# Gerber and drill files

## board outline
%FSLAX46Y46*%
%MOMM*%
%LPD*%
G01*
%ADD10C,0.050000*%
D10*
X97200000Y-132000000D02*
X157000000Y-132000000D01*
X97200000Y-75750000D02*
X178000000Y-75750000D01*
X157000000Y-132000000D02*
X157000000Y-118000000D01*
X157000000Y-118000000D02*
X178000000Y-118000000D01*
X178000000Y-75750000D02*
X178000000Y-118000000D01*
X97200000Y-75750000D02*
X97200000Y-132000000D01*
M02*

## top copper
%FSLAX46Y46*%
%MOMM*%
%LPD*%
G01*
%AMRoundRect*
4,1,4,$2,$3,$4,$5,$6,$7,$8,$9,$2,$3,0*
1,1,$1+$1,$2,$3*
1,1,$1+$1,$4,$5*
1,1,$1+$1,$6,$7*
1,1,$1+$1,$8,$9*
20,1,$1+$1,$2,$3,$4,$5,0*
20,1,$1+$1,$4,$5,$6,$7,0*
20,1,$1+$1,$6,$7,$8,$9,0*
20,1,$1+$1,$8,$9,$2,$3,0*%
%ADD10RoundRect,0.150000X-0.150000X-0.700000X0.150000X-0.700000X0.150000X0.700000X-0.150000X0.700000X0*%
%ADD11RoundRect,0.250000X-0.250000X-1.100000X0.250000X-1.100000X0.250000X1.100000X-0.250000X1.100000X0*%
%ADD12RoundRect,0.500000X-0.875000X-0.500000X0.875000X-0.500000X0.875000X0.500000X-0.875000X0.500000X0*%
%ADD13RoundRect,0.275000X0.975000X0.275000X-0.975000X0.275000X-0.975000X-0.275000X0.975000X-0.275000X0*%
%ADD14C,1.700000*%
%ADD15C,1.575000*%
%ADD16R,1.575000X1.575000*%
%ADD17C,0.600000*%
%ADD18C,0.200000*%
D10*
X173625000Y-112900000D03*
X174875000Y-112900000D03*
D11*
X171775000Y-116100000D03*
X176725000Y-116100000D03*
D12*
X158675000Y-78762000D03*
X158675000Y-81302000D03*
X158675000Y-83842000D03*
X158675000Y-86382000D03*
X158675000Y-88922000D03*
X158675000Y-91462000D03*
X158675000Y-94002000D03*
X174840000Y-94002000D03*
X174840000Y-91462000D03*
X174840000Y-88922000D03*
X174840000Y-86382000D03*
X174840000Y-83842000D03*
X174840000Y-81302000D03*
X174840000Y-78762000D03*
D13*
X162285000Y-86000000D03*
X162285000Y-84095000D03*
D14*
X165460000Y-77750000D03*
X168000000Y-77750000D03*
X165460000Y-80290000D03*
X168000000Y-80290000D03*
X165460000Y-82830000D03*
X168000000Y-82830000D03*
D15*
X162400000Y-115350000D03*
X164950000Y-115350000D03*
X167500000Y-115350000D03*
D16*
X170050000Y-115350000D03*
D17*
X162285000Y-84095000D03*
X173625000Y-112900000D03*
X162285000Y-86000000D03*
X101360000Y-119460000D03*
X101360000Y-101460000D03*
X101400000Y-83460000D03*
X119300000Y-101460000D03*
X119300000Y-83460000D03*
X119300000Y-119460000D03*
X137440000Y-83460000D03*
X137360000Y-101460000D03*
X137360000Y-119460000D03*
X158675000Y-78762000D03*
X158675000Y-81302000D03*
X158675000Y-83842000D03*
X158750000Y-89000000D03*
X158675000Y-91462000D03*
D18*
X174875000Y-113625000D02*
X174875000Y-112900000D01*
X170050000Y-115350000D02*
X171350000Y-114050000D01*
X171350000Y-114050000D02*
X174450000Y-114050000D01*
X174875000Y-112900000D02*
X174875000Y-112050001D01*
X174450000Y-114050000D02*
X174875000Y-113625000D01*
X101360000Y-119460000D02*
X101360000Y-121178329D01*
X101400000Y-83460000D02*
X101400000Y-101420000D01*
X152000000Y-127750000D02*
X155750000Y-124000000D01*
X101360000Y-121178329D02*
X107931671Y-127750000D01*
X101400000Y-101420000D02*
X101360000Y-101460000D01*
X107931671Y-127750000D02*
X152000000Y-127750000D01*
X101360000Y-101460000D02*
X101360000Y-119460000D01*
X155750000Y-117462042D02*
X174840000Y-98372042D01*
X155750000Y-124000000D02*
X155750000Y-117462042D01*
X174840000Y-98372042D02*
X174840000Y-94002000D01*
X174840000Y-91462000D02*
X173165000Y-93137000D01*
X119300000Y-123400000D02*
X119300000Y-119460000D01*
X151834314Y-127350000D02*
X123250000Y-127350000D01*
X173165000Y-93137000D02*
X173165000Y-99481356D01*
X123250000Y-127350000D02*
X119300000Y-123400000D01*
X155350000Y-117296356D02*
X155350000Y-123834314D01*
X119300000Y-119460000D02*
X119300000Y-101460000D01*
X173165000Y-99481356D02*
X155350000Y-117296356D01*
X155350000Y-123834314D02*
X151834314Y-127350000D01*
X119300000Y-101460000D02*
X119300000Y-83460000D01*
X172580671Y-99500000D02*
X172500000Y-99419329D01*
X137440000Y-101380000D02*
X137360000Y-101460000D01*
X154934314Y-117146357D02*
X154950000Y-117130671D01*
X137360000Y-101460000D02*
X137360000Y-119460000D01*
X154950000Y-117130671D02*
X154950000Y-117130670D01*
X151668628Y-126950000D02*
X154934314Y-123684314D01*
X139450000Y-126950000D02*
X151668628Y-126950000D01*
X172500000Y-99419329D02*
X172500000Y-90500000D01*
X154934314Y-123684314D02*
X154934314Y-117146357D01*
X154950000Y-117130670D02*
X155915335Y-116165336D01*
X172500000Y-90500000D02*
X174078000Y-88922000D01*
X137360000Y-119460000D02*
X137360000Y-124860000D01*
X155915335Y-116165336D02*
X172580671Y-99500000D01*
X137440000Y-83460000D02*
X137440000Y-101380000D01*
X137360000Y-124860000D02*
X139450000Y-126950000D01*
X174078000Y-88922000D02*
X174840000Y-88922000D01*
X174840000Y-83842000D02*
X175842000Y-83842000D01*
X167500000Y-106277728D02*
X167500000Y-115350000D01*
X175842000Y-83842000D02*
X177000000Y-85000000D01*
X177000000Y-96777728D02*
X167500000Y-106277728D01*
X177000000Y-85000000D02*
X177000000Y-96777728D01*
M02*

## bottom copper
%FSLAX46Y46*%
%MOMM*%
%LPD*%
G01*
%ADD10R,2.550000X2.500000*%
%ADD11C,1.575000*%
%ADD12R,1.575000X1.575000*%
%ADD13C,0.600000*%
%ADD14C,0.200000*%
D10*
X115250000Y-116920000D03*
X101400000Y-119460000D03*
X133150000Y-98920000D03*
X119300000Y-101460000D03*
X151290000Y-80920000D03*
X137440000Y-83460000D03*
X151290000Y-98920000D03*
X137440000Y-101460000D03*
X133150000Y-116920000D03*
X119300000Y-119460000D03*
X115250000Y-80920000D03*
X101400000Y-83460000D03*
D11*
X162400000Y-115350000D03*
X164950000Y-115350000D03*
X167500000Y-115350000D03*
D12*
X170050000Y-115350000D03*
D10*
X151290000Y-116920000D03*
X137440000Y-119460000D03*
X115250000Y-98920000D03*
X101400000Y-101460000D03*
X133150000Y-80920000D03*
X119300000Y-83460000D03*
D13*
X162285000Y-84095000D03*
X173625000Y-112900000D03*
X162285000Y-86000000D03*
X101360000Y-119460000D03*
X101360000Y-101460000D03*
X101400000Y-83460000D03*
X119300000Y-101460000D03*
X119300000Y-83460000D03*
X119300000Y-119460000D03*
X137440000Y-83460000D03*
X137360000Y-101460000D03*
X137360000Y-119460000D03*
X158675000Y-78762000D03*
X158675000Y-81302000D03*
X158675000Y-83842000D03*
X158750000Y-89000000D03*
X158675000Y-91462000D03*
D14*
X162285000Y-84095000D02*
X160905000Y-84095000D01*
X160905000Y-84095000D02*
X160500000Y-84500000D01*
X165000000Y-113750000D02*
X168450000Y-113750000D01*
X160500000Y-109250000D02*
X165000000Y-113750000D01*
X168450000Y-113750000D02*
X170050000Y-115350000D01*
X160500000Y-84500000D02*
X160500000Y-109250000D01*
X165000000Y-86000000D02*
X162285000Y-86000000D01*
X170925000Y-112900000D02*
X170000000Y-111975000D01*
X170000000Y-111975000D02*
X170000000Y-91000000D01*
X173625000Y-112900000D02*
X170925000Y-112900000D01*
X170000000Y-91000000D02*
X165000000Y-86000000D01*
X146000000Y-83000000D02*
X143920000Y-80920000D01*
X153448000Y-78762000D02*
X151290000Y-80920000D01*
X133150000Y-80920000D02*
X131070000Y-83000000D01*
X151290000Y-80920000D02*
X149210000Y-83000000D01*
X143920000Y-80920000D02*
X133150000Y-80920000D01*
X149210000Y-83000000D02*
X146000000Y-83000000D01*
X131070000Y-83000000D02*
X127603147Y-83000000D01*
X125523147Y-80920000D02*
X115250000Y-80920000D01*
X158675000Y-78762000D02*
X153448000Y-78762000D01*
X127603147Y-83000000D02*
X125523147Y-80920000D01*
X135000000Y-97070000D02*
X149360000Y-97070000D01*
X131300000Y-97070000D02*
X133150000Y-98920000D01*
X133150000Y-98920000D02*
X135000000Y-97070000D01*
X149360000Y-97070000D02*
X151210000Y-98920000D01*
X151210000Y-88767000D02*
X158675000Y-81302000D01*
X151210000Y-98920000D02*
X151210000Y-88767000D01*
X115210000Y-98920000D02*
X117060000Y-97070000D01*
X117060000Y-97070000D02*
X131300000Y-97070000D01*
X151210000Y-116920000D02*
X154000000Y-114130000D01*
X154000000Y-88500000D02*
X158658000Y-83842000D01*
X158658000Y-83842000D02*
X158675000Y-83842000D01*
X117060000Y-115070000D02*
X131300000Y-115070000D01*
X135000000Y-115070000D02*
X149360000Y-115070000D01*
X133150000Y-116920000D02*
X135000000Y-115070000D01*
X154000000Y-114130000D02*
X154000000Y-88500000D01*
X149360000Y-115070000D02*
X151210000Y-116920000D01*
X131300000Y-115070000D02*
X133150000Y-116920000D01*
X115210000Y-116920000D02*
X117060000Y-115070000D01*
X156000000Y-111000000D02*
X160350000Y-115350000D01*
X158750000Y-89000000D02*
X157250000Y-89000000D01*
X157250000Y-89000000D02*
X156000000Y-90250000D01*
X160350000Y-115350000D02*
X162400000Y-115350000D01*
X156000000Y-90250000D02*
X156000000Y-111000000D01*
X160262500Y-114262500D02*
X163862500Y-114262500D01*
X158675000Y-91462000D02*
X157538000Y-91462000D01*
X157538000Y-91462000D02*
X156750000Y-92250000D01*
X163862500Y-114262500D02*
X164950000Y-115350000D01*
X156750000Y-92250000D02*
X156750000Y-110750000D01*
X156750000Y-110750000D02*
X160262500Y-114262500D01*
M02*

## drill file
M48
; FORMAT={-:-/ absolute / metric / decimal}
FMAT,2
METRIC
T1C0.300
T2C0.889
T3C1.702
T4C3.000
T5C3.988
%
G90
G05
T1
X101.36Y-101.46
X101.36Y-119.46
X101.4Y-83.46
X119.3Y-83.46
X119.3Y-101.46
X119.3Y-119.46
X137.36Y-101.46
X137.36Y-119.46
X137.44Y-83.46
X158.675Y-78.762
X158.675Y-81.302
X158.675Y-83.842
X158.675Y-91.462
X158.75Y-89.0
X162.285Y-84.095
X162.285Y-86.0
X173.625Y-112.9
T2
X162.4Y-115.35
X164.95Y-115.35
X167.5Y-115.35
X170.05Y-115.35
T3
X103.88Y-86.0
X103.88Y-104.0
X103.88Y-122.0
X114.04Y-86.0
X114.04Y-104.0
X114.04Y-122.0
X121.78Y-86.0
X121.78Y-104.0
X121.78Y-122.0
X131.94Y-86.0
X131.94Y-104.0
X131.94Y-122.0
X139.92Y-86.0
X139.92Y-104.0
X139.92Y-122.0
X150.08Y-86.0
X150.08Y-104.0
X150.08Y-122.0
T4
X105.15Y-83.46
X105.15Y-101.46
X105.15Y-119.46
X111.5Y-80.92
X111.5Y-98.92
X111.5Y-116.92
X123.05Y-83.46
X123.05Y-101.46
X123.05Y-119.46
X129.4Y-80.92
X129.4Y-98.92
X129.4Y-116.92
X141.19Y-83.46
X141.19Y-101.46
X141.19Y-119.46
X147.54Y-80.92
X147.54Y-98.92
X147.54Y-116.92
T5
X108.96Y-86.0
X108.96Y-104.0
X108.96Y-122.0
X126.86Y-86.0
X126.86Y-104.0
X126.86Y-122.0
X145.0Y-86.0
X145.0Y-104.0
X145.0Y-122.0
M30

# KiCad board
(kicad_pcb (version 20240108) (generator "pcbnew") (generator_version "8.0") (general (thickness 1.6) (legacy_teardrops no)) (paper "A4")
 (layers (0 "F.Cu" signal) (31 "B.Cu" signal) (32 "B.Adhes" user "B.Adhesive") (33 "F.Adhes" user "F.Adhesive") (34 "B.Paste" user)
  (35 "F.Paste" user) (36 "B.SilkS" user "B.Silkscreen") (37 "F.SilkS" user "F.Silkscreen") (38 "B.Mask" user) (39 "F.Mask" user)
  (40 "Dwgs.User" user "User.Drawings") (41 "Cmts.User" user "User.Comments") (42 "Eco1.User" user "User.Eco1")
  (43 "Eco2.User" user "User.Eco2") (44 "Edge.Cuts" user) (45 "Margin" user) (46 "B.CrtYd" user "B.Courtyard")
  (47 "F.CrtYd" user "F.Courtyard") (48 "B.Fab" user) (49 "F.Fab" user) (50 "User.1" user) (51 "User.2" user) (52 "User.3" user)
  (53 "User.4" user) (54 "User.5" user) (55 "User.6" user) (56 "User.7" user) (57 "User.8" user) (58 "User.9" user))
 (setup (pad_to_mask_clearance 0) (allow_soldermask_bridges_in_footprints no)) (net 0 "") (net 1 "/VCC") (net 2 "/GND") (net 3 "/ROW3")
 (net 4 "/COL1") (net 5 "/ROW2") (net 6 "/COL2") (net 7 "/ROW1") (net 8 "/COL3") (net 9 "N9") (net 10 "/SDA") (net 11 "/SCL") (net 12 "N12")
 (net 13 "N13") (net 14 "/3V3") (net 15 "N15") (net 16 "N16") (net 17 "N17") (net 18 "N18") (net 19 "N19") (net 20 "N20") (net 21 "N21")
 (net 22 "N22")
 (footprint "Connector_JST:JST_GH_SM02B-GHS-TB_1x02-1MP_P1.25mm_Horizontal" (layer "F.Cu") (at 174.25 114.75)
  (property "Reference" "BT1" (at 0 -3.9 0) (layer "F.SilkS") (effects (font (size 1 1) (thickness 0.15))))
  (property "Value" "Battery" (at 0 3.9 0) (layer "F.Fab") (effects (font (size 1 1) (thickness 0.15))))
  (pad "1" smd roundrect (at -0.625 -1.85) (size 0.6 1.7) (layers "F.Cu" "F.Paste" "F.Mask") (roundrect_rratio 0.25) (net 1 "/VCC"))
  (pad "2" smd roundrect (at 0.625 -1.85) (size 0.6 1.7) (layers "F.Cu" "F.Paste" "F.Mask") (roundrect_rratio 0.25) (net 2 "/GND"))
  (pad "MP" smd roundrect (at -2.475 1.35) (size 1 2.7) (layers "F.Cu" "F.Paste" "F.Mask") (roundrect_rratio 0.25))
  (pad "MP" smd roundrect (at 2.475 1.35) (size 1 2.7) (layers "F.Cu" "F.Paste" "F.Mask") (roundrect_rratio 0.25)))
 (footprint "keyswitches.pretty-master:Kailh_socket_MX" (layer "F.Cu") (at 108.96 122)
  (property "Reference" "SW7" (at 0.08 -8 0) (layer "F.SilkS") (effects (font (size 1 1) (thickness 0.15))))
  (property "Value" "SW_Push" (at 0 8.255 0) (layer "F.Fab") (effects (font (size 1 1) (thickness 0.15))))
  (pad "" np_thru_hole circle (at -5.08 0) (size 1.7018 1.7018) (drill 1.7018) (layers "*.Cu" "*.Mask"))
  (pad "" np_thru_hole circle (at -3.81 -2.54) (size 3 3) (drill 3) (layers "*.Cu" "*.Mask"))
  (pad "" np_thru_hole circle (at 0 0) (size 3.9878 3.9878) (drill 3.9878) (layers "*.Cu" "*.Mask"))
  (pad "" np_thru_hole circle (at 2.54 -5.08) (size 3 3) (drill 3) (layers "*.Cu" "*.Mask"))
  (pad "" np_thru_hole circle (at 5.08 0) (size 1.7018 1.7018) (drill 1.7018) (layers "*.Cu" "*.Mask"))
  (pad "1" smd rect (at 6.29 -5.08) (size 2.55 2.5) (layers "B.Cu" "B.Paste" "B.Mask") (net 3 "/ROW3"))
  (pad "2" smd rect (at -7.56 -2.54) (size 2.55 2.5) (layers "B.Cu" "B.Paste" "B.Mask") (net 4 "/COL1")))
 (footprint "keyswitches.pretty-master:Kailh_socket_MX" (layer "F.Cu") (at 126.86 104)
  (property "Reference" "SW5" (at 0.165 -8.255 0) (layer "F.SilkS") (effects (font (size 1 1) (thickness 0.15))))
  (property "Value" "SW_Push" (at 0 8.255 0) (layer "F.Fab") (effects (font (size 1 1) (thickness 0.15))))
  (pad "" np_thru_hole circle (at -5.08 0) (size 1.7018 1.7018) (drill 1.7018) (layers "*.Cu" "*.Mask"))
  (pad "" np_thru_hole circle (at -3.81 -2.54) (size 3 3) (drill 3) (layers "*.Cu" "*.Mask"))
  (pad "" np_thru_hole circle (at 0 0) (size 3.9878 3.9878) (drill 3.9878) (layers "*.Cu" "*.Mask"))
  (pad "" np_thru_hole circle (at 2.54 -5.08) (size 3 3) (drill 3) (layers "*.Cu" "*.Mask"))
  (pad "" np_thru_hole circle (at 5.08 0) (size 1.7018 1.7018) (drill 1.7018) (layers "*.Cu" "*.Mask"))
  (pad "1" smd rect (at 6.29 -5.08) (size 2.55 2.5) (layers "B.Cu" "B.Paste" "B.Mask") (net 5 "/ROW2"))
  (pad "2" smd rect (at -7.56 -2.54) (size 2.55 2.5) (layers "B.Cu" "B.Paste" "B.Mask") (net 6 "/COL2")))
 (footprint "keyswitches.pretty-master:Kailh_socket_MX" (layer "F.Cu") (at 145 86)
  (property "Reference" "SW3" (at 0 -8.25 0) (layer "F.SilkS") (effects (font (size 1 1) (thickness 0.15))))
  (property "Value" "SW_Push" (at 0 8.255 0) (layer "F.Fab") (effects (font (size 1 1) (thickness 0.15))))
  (pad "" np_thru_hole circle (at -5.08 0) (size 1.7018 1.7018) (drill 1.7018) (layers "*.Cu" "*.Mask"))
  (pad "" np_thru_hole circle (at -3.81 -2.54) (size 3 3) (drill 3) (layers "*.Cu" "*.Mask"))
  (pad "" np_thru_hole circle (at 0 0) (size 3.9878 3.9878) (drill 3.9878) (layers "*.Cu" "*.Mask"))
  (pad "" np_thru_hole circle (at 2.54 -5.08) (size 3 3) (drill 3) (layers "*.Cu" "*.Mask"))
  (pad "" np_thru_hole circle (at 5.08 0) (size 1.7018 1.7018) (drill 1.7018) (layers "*.Cu" "*.Mask"))
  (pad "1" smd rect (at 6.29 -5.08) (size 2.55 2.5) (layers "B.Cu" "B.Paste" "B.Mask") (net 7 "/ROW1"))
  (pad "2" smd rect (at -7.56 -2.54) (size 2.55 2.5) (layers "B.Cu" "B.Paste" "B.Mask") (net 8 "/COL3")))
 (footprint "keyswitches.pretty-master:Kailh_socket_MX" (layer "F.Cu") (at 145 104)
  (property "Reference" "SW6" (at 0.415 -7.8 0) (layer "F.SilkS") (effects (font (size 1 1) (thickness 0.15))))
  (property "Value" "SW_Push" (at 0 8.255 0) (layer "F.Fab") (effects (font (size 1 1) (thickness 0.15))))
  (pad "" np_thru_hole circle (at -5.08 0) (size 1.7018 1.7018) (drill 1.7018) (layers "*.Cu" "*.Mask"))
  (pad "" np_thru_hole circle (at -3.81 -2.54) (size 3 3) (drill 3) (layers "*.Cu" "*.Mask"))
  (pad "" np_thru_hole circle (at 0 0) (size 3.9878 3.9878) (drill 3.9878) (layers "*.Cu" "*.Mask"))
  (pad "" np_thru_hole circle (at 2.54 -5.08) (size 3 3) (drill 3) (layers "*.Cu" "*.Mask"))
  (pad "" np_thru_hole circle (at 5.08 0) (size 1.7018 1.7018) (drill 1.7018) (layers "*.Cu" "*.Mask"))
  (pad "1" smd rect (at 6.29 -5.08) (size 2.55 2.5) (layers "B.Cu" "B.Paste" "B.Mask") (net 5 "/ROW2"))
  (pad "2" smd rect (at -7.56 -2.54) (size 2.55 2.5) (layers "B.Cu" "B.Paste" "B.Mask") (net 8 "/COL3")))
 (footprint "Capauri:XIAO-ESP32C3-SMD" (layer "F.Cu") (at 166.675 86.342)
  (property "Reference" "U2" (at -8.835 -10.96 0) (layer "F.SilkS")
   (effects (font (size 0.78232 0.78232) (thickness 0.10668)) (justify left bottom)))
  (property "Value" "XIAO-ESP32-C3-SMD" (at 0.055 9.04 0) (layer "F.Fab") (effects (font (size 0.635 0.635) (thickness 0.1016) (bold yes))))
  (pad "1" smd roundrect (at -8 -7.58) (size 2.75 2) (layers "F.Cu" "F.Paste" "F.Mask") (roundrect_rratio 0.25) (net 7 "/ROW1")
   (solder_mask_margin 0.0508) (thermal_bridge_angle 45))
  (pad "2" smd roundrect (at -8 -5.04) (size 2.75 2) (layers "F.Cu" "F.Paste" "F.Mask") (roundrect_rratio 0.25) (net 5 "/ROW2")
   (solder_mask_margin 0.0508) (thermal_bridge_angle 45))
  (pad "3" smd roundrect (at -8 -2.5) (size 2.75 2) (layers "F.Cu" "F.Paste" "F.Mask") (roundrect_rratio 0.25) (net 3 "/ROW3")
   (solder_mask_margin 0.0508) (thermal_bridge_angle 45))
  (pad "4" smd roundrect (at -8 0.04) (size 2.75 2) (layers "F.Cu" "F.Paste" "F.Mask") (roundrect_rratio 0.25) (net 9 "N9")
   (solder_mask_margin 0.0508) (thermal_bridge_angle 45))
  (pad "5" smd roundrect (at -8 2.58) (size 2.75 2) (layers "F.Cu" "F.Paste" "F.Mask") (roundrect_rratio 0.25) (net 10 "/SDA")
   (solder_mask_margin 0.0508) (thermal_bridge_angle 45))
  (pad "6" smd roundrect (at -8 5.12) (size 2.75 2) (layers "F.Cu" "F.Paste" "F.Mask") (roundrect_rratio 0.25) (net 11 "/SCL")
   (solder_mask_margin 0.0508) (thermal_bridge_angle 45))
  (pad "7" smd roundrect (at -8 7.66) (size 2.75 2) (layers "F.Cu" "F.Paste" "F.Mask") (roundrect_rratio 0.25) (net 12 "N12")
   (solder_mask_margin 0.0508) (thermal_bridge_angle 45))
  (pad "8" smd roundrect (at 8.165 7.66) (size 2.75 2) (layers "F.Cu" "F.Paste" "F.Mask") (roundrect_rratio 0.25) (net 4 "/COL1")
   (solder_mask_margin 0.0508) (thermal_bridge_angle 45))
  (pad "9" smd roundrect (at 8.165 5.12) (size 2.75 2) (layers "F.Cu" "F.Paste" "F.Mask") (roundrect_rratio 0.25) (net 6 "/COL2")
   (solder_mask_margin 0.0508) (thermal_bridge_angle 45))
  (pad "10" smd roundrect (at 8.165 2.58) (size 2.75 2) (layers "F.Cu" "F.Paste" "F.Mask") (roundrect_rratio 0.25) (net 8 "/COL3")
   (solder_mask_margin 0.0508) (thermal_bridge_angle 45))
  (pad "11" smd roundrect (at 8.165 0.04) (size 2.75 2) (layers "F.Cu" "F.Paste" "F.Mask") (roundrect_rratio 0.25) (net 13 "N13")
   (solder_mask_margin 0.0508) (thermal_bridge_angle 45))
  (pad "12" smd roundrect (at 8.165 -2.5) (size 2.75 2) (layers "F.Cu" "F.Paste" "F.Mask") (roundrect_rratio 0.25) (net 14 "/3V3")
   (solder_mask_margin 0.0508) (thermal_bridge_angle 45))
  (pad "13" smd roundrect (at 8.165 -5.04) (size 2.75 2) (layers "F.Cu" "F.Paste" "F.Mask") (roundrect_rratio 0.25) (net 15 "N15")
   (solder_mask_margin 0.0508) (thermal_bridge_angle 45))
  (pad "14" smd roundrect (at 8.165 -7.58) (size 2.75 2) (layers "F.Cu" "F.Paste" "F.Mask") (roundrect_rratio 0.25) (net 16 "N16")
   (solder_mask_margin 0.0508) (thermal_bridge_angle 45))
  (pad "15" smd roundrect (at -4.39 -0.342 180) (size 2.5 1.1) (layers "F.Cu" "F.Paste" "F.Mask") (roundrect_rratio 0.25) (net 1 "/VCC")
   (solder_mask_margin 0.0508) (thermal_bridge_angle 45))
  (pad "16" smd roundrect (at -4.39 -2.247 180) (size 2.5 1.1) (layers "F.Cu" "F.Paste" "F.Mask") (roundrect_rratio 0.25) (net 2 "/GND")
   (solder_mask_margin 0.0508) (thermal_bridge_angle 45))
  (pad "17" smd circle (at -1.215 -8.592) (size 1.7 1.7) (layers "F.Cu" "F.Paste" "F.Mask") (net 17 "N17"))
  (pad "18" smd circle (at 1.325 -8.592) (size 1.7 1.7) (layers "F.Cu" "F.Paste" "F.Mask") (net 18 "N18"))
  (pad "19" smd circle (at -1.215 -6.052) (size 1.7 1.7) (layers "F.Cu" "F.Paste" "F.Mask") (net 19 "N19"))
  (pad "20" smd circle (at 1.325 -6.052) (size 1.7 1.7) (layers "F.Cu" "F.Paste" "F.Mask") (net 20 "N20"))
  (pad "21" smd circle (at -1.215 -3.512) (size 1.7 1.7) (layers "F.Cu" "F.Paste" "F.Mask") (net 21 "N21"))
  (pad "22" smd circle (at 1.325 -3.512) (size 1.7 1.7) (layers "F.Cu" "F.Paste" "F.Mask") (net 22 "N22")))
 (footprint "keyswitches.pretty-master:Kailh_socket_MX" (layer "F.Cu") (at 126.86 122)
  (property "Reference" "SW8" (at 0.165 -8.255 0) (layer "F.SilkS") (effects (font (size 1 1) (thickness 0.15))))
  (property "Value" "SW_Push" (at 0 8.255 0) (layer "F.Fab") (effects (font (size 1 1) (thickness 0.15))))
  (pad "" np_thru_hole circle (at -5.08 0) (size 1.7018 1.7018) (drill 1.7018) (layers "*.Cu" "*.Mask"))
  (pad "" np_thru_hole circle (at -3.81 -2.54) (size 3 3) (drill 3) (layers "*.Cu" "*.Mask"))
  (pad "" np_thru_hole circle (at 0 0) (size 3.9878 3.9878) (drill 3.9878) (layers "*.Cu" "*.Mask"))
  (pad "" np_thru_hole circle (at 2.54 -5.08) (size 3 3) (drill 3) (layers "*.Cu" "*.Mask"))
  (pad "" np_thru_hole circle (at 5.08 0) (size 1.7018 1.7018) (drill 1.7018) (layers "*.Cu" "*.Mask"))
  (pad "1" smd rect (at 6.29 -5.08) (size 2.55 2.5) (layers "B.Cu" "B.Paste" "B.Mask") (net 3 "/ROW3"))
  (pad "2" smd rect (at -7.56 -2.54) (size 2.55 2.5) (layers "B.Cu" "B.Paste" "B.Mask") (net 6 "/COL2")))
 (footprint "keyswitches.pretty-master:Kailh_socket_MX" (layer "F.Cu") (at 108.96 86)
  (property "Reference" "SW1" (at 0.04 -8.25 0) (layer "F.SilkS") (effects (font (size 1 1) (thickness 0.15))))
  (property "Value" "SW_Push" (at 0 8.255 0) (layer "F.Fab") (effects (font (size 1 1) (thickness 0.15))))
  (pad "" np_thru_hole circle (at -5.08 0) (size 1.7018 1.7018) (drill 1.7018) (layers "*.Cu" "*.Mask"))
  (pad "" np_thru_hole circle (at -3.81 -2.54) (size 3 3) (drill 3) (layers "*.Cu" "*.Mask"))
  (pad "" np_thru_hole circle (at 0 0) (size 3.9878 3.9878) (drill 3.9878) (layers "*.Cu" "*.Mask"))
  (pad "" np_thru_hole circle (at 2.54 -5.08) (size 3 3) (drill 3) (layers "*.Cu" "*.Mask"))
  (pad "" np_thru_hole circle (at 5.08 0) (size 1.7018 1.7018) (drill 1.7018) (layers "*.Cu" "*.Mask"))
  (pad "1" smd rect (at 6.29 -5.08) (size 2.55 2.5) (layers "B.Cu" "B.Paste" "B.Mask") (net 7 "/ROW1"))
  (pad "2" smd rect (at -7.56 -2.54) (size 2.55 2.5) (layers "B.Cu" "B.Paste" "B.Mask") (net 4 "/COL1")))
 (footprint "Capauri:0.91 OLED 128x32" (layer "F.Cu") (at 166.25 121.9)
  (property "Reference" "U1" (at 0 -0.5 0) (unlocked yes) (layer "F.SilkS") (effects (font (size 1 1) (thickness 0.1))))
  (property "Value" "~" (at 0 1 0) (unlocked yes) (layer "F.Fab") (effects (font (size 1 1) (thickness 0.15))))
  (pad "1" thru_hole circle (at -3.85 -6.55) (size 1.575 1.575) (drill 0.889) (layers "*.Cu" "*.Mask") (remove_unused_layers no)
   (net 10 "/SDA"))
  (pad "2" thru_hole circle (at -1.3 -6.55) (size 1.575 1.575) (drill 0.889) (layers "*.Cu" "*.Mask") (remove_unused_layers no)
   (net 11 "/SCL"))
  (pad "3" thru_hole circle (at 1.25 -6.55) (size 1.575 1.575) (drill 0.889) (layers "*.Cu" "*.Mask") (remove_unused_layers no)
   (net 14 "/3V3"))
  (pad "4" thru_hole rect (at 3.8 -6.55) (size 1.575 1.575) (drill 0.889) (layers "*.Cu" "*.Mask") (remove_unused_layers no) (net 2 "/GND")
   (thermal_bridge_angle 45)))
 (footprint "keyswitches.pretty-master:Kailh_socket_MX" (layer "F.Cu") (at 145 122)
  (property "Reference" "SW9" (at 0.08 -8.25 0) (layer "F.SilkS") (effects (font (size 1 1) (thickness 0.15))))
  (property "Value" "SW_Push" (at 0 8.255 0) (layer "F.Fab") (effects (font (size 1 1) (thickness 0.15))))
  (pad "" np_thru_hole circle (at -5.08 0) (size 1.7018 1.7018) (drill 1.7018) (layers "*.Cu" "*.Mask"))
  (pad "" np_thru_hole circle (at -3.81 -2.54) (size 3 3) (drill 3) (layers "*.Cu" "*.Mask"))
  (pad "" np_thru_hole circle (at 0 0) (size 3.9878 3.9878) (drill 3.9878) (layers "*.Cu" "*.Mask"))
  (pad "" np_thru_hole circle (at 2.54 -5.08) (size 3 3) (drill 3) (layers "*.Cu" "*.Mask"))
  (pad "" np_thru_hole circle (at 5.08 0) (size 1.7018 1.7018) (drill 1.7018) (layers "*.Cu" "*.Mask"))
  (pad "1" smd rect (at 6.29 -5.08) (size 2.55 2.5) (layers "B.Cu" "B.Paste" "B.Mask") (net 3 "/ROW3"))
  (pad "2" smd rect (at -7.56 -2.54) (size 2.55 2.5) (layers "B.Cu" "B.Paste" "B.Mask") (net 8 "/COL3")))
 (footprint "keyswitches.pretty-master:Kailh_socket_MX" (layer "F.Cu") (at 108.96 104)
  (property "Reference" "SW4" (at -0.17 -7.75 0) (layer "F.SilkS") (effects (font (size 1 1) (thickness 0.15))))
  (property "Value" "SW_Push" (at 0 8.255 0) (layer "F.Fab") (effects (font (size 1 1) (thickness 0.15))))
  (pad "" np_thru_hole circle (at -5.08 0) (size 1.7018 1.7018) (drill 1.7018) (layers "*.Cu" "*.Mask"))
  (pad "" np_thru_hole circle (at -3.81 -2.54) (size 3 3) (drill 3) (layers "*.Cu" "*.Mask"))
  (pad "" np_thru_hole circle (at 0 0) (size 3.9878 3.9878) (drill 3.9878) (layers "*.Cu" "*.Mask"))
  (pad "" np_thru_hole circle (at 2.54 -5.08) (size 3 3) (drill 3) (layers "*.Cu" "*.Mask"))
  (pad "" np_thru_hole circle (at 5.08 0) (size 1.7018 1.7018) (drill 1.7018) (layers "*.Cu" "*.Mask"))
  (pad "1" smd rect (at 6.29 -5.08) (size 2.55 2.5) (layers "B.Cu" "B.Paste" "B.Mask") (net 5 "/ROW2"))
  (pad "2" smd rect (at -7.56 -2.54) (size 2.55 2.5) (layers "B.Cu" "B.Paste" "B.Mask") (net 4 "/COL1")))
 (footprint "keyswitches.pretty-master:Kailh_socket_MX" (layer "F.Cu") (at 126.86 86)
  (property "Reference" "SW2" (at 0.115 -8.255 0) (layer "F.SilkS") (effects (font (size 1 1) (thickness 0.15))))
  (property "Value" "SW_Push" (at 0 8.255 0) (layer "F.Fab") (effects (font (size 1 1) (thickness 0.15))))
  (pad "" np_thru_hole circle (at -5.08 0) (size 1.7018 1.7018) (drill 1.7018) (layers "*.Cu" "*.Mask"))
  (pad "" np_thru_hole circle (at -3.81 -2.54) (size 3 3) (drill 3) (layers "*.Cu" "*.Mask"))
  (pad "" np_thru_hole circle (at 0 0) (size 3.9878 3.9878) (drill 3.9878) (layers "*.Cu" "*.Mask"))
  (pad "" np_thru_hole circle (at 2.54 -5.08) (size 3 3) (drill 3) (layers "*.Cu" "*.Mask"))
  (pad "" np_thru_hole circle (at 5.08 0) (size 1.7018 1.7018) (drill 1.7018) (layers "*.Cu" "*.Mask"))
  (pad "1" smd rect (at 6.29 -5.08) (size 2.55 2.5) (layers "B.Cu" "B.Paste" "B.Mask") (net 7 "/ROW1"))
  (pad "2" smd rect (at -7.56 -2.54) (size 2.55 2.5) (layers "B.Cu" "B.Paste" "B.Mask") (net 6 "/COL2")))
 (gr_line (start 97.2 132) (end 157 132) (stroke (width 0.05) (type default)) (layer "Edge.Cuts"))
 (gr_line (start 97.2 75.75) (end 178 75.75) (stroke (width 0.05) (type default)) (layer "Edge.Cuts"))
 (gr_line (start 157 132) (end 157 118) (stroke (width 0.05) (type default)) (layer "Edge.Cuts"))
 (gr_line (start 157 118) (end 178 118) (stroke (width 0.05) (type default)) (layer "Edge.Cuts"))
 (gr_line (start 178 75.75) (end 178 118) (stroke (width 0.05) (type default)) (layer "Edge.Cuts"))
 (gr_line (start 97.2 75.75) (end 97.2 132) (stroke (width 0.05) (type default)) (layer "Edge.Cuts"))
 (segment (start 174.875 113.625) (end 174.875 112.9) (width 0.2) (layer "F.Cu") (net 2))
 (segment (start 170.05 115.35) (end 171.35 114.05) (width 0.2) (layer "F.Cu") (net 2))
 (segment (start 171.35 114.05) (end 174.45 114.05) (width 0.2) (layer "F.Cu") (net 2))
 (segment (start 174.875 112.9) (end 174.875 112.050001) (width 0.2) (layer "F.Cu") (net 2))
 (segment (start 174.45 114.05) (end 174.875 113.625) (width 0.2) (layer "F.Cu") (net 2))
 (via (at 162.285 84.095) (size 0.6) (drill 0.3) (layers "F.Cu" "B.Cu") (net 2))
 (segment (start 162.285 84.095) (end 160.905 84.095) (width 0.2) (layer "B.Cu") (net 2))
 (segment (start 160.905 84.095) (end 160.5 84.5) (width 0.2) (layer "B.Cu") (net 2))
 (segment (start 165 113.75) (end 168.45 113.75) (width 0.2) (layer "B.Cu") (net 2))
 (segment (start 160.5 109.25) (end 165 113.75) (width 0.2) (layer "B.Cu") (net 2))
 (segment (start 168.45 113.75) (end 170.05 115.35) (width 0.2) (layer "B.Cu") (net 2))
 (segment (start 160.5 84.5) (end 160.5 109.25) (width 0.2) (layer "B.Cu") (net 2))
 (via (at 173.625 112.9) (size 0.6) (drill 0.3) (layers "F.Cu" "B.Cu") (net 1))
 (via (at 162.285 86) (size 0.6) (drill 0.3) (layers "F.Cu" "B.Cu") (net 1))
 (segment (start 165 86) (end 162.285 86) (width 0.2) (layer "B.Cu") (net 1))
 (segment (start 170.925 112.9) (end 170 111.975) (width 0.2) (layer "B.Cu") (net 1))
 (segment (start 170 111.975) (end 170 91) (width 0.2) (layer "B.Cu") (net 1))
 (segment (start 173.625 112.9) (end 170.925 112.9) (width 0.2) (layer "B.Cu") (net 1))
 (segment (start 170 91) (end 165 86) (width 0.2) (layer "B.Cu") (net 1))
 (segment (start 101.36 119.46) (end 101.36 121.178329) (width 0.2) (layer "F.Cu") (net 4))
 (segment (start 101.4 83.46) (end 101.4 101.42) (width 0.2) (layer "F.Cu") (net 4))
 (segment (start 152 127.75) (end 155.75 124) (width 0.2) (layer "F.Cu") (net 4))
 (segment (start 101.36 121.178329) (end 107.931671 127.75) (width 0.2) (layer "F.Cu") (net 4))
 (segment (start 101.4 101.42) (end 101.36 101.46) (width 0.2) (layer "F.Cu") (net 4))
 (segment (start 107.931671 127.75) (end 152 127.75) (width 0.2) (layer "F.Cu") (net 4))
 (segment (start 101.36 101.46) (end 101.36 119.46) (width 0.2) (layer "F.Cu") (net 4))
 (segment (start 155.75 117.462042) (end 174.84 98.372042) (width 0.2) (layer "F.Cu") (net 4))
 (segment (start 155.75 124) (end 155.75 117.462042) (width 0.2) (layer "F.Cu") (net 4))
 (segment (start 174.84 98.372042) (end 174.84 94.002) (width 0.2) (layer "F.Cu") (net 4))
 (via (at 101.36 119.46) (size 0.6) (drill 0.3) (layers "F.Cu" "B.Cu") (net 4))
 (via (at 101.36 101.46) (size 0.6) (drill 0.3) (layers "F.Cu" "B.Cu") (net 4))
 (via (at 101.4 83.46) (size 0.6) (drill 0.3) (layers "F.Cu" "B.Cu") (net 4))
 (segment (start 174.84 91.462) (end 173.165 93.137) (width 0.2) (layer "F.Cu") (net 6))
 (segment (start 119.3 123.4) (end 119.3 119.46) (width 0.2) (layer "F.Cu") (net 6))
 (segment (start 151.834314 127.35) (end 123.25 127.35) (width 0.2) (layer "F.Cu") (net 6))
 (segment (start 173.165 93.137) (end 173.165 99.481356) (width 0.2) (layer "F.Cu") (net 6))
 (segment (start 123.25 127.35) (end 119.3 123.4) (width 0.2) (layer "F.Cu") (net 6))
 (segment (start 155.35 117.296356) (end 155.35 123.834314) (width 0.2) (layer "F.Cu") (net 6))
 (segment (start 119.3 119.46) (end 119.3 101.46) (width 0.2) (layer "F.Cu") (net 6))
 (segment (start 173.165 99.481356) (end 155.35 117.296356) (width 0.2) (layer "F.Cu") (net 6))
 (segment (start 155.35 123.834314) (end 151.834314 127.35) (width 0.2) (layer "F.Cu") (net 6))
 (segment (start 119.3 101.46) (end 119.3 83.46) (width 0.2) (layer "F.Cu") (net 6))
 (via (at 119.3 101.46) (size 0.6) (drill 0.3) (layers "F.Cu" "B.Cu") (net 6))
 (via (at 119.3 83.46) (size 0.6) (drill 0.3) (layers "F.Cu" "B.Cu") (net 6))
 (via (at 119.3 119.46) (size 0.6) (drill 0.3) (layers "F.Cu" "B.Cu") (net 6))
 (segment (start 172.580671 99.5) (end 172.5 99.419329) (width 0.2) (layer "F.Cu") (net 8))
 (segment (start 137.44 101.38) (end 137.36 101.46) (width 0.2) (layer "F.Cu") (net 8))
 (segment (start 154.934314 117.146357) (end 154.95 117.130671) (width 0.2) (layer "F.Cu") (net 8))
 (segment (start 137.36 101.46) (end 137.36 119.46) (width 0.2) (layer "F.Cu") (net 8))
 (segment (start 154.95 117.130671) (end 154.95 117.13067) (width 0.2) (layer "F.Cu") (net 8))
 (segment (start 151.668628 126.95) (end 154.934314 123.684314) (width 0.2) (layer "F.Cu") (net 8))
 (segment (start 139.45 126.95) (end 151.668628 126.95) (width 0.2) (layer "F.Cu") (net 8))
 (segment (start 172.5 99.419329) (end 172.5 90.5) (width 0.2) (layer "F.Cu") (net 8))
 (segment (start 154.934314 123.684314) (end 154.934314 117.146357) (width 0.2) (layer "F.Cu") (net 8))
 (segment (start 154.95 117.13067) (end 155.915335 116.165336) (width 0.2) (layer "F.Cu") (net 8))
 (segment (start 172.5 90.5) (end 174.078 88.922) (width 0.2) (layer "F.Cu") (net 8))
 (segment (start 137.36 119.46) (end 137.36 124.86) (width 0.2) (layer "F.Cu") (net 8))
 (segment (start 155.915335 116.165336) (end 172.580671 99.5) (width 0.2) (layer "F.Cu") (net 8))
 (segment (start 137.44 83.46) (end 137.44 101.38) (width 0.2) (layer "F.Cu") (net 8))
 (segment (start 137.36 124.86) (end 139.45 126.95) (width 0.2) (layer "F.Cu") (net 8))
 (segment (start 174.078 88.922) (end 174.84 88.922) (width 0.2) (layer "F.Cu") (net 8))
 (via (at 137.44 83.46) (size 0.6) (drill 0.3) (layers "F.Cu" "B.Cu") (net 8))
 (via (at 137.36 101.46) (size 0.6) (drill 0.3) (layers "F.Cu" "B.Cu") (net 8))
 (via (at 137.36 119.46) (size 0.6) (drill 0.3) (layers "F.Cu" "B.Cu") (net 8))
 (segment (start 174.84 83.842) (end 175.842 83.842) (width 0.2) (layer "F.Cu") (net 14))
 (segment (start 167.5 106.277728) (end 167.5 115.35) (width 0.2) (layer "F.Cu") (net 14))
 (segment (start 175.842 83.842) (end 177 85) (width 0.2) (layer "F.Cu") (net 14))
 (segment (start 177 96.777728) (end 167.5 106.277728) (width 0.2) (layer "F.Cu") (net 14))
 (segment (start 177 85) (end 177 96.777728) (width 0.2) (layer "F.Cu") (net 14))
 (via (at 158.675 78.762) (size 0.6) (drill 0.3) (layers "F.Cu" "B.Cu") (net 7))
 (segment (start 146 83) (end 143.92 80.92) (width 0.2) (layer "B.Cu") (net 7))
 (segment (start 153.448 78.762) (end 151.29 80.92) (width 0.2) (layer "B.Cu") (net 7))
 (segment (start 133.15 80.92) (end 131.07 83) (width 0.2) (layer "B.Cu") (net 7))
 (segment (start 151.29 80.92) (end 149.21 83) (width 0.2) (layer "B.Cu") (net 7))
 (segment (start 143.92 80.92) (end 133.15 80.92) (width 0.2) (layer "B.Cu") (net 7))
 (segment (start 149.21 83) (end 146 83) (width 0.2) (layer "B.Cu") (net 7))
 (segment (start 131.07 83) (end 127.603147 83) (width 0.2) (layer "B.Cu") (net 7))
 (segment (start 125.523147 80.92) (end 115.25 80.92) (width 0.2) (layer "B.Cu") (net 7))
 (segment (start 158.675 78.762) (end 153.448 78.762) (width 0.2) (layer "B.Cu") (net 7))
 (segment (start 127.603147 83) (end 125.523147 80.92) (width 0.2) (layer "B.Cu") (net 7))
 (via (at 158.675 81.302) (size 0.6) (drill 0.3) (layers "F.Cu" "B.Cu") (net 5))
 (segment (start 135 97.07) (end 149.36 97.07) (width 0.2) (layer "B.Cu") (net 5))
 (segment (start 131.3 97.07) (end 133.15 98.92) (width 0.2) (layer "B.Cu") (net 5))
 (segment (start 133.15 98.92) (end 135 97.07) (width 0.2) (layer "B.Cu") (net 5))
 (segment (start 149.36 97.07) (end 151.21 98.92) (width 0.2) (layer "B.Cu") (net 5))
 (segment (start 151.21 88.767) (end 158.675 81.302) (width 0.2) (layer "B.Cu") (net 5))
 (segment (start 151.21 98.92) (end 151.21 88.767) (width 0.2) (layer "B.Cu") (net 5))
 (segment (start 115.21 98.92) (end 117.06 97.07) (width 0.2) (layer "B.Cu") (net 5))
 (segment (start 117.06 97.07) (end 131.3 97.07) (width 0.2) (layer "B.Cu") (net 5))
 (via (at 158.675 83.842) (size 0.6) (drill 0.3) (layers "F.Cu" "B.Cu") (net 3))
 (segment (start 151.21 116.92) (end 154 114.13) (width 0.2) (layer "B.Cu") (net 3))
 (segment (start 154 88.5) (end 158.658 83.842) (width 0.2) (layer "B.Cu") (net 3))
 (segment (start 158.658 83.842) (end 158.675 83.842) (width 0.2) (layer "B.Cu") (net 3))
 (segment (start 117.06 115.07) (end 131.3 115.07) (width 0.2) (layer "B.Cu") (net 3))
 (segment (start 135 115.07) (end 149.36 115.07) (width 0.2) (layer "B.Cu") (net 3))
 (segment (start 133.15 116.92) (end 135 115.07) (width 0.2) (layer "B.Cu") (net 3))
 (segment (start 154 114.13) (end 154 88.5) (width 0.2) (layer "B.Cu") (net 3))
 (segment (start 149.36 115.07) (end 151.21 116.92) (width 0.2) (layer "B.Cu") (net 3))
 (segment (start 131.3 115.07) (end 133.15 116.92) (width 0.2) (layer "B.Cu") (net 3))
 (segment (start 115.21 116.92) (end 117.06 115.07) (width 0.2) (layer "B.Cu") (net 3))
 (via (at 158.75 89) (size 0.6) (drill 0.3) (layers "F.Cu" "B.Cu") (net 10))
 (segment (start 156 111) (end 160.35 115.35) (width 0.2) (layer "B.Cu") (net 10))
 (segment (start 158.75 89) (end 157.25 89) (width 0.2) (layer "B.Cu") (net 10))
 (segment (start 157.25 89) (end 156 90.25) (width 0.2) (layer "B.Cu") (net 10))
 (segment (start 160.35 115.35) (end 162.4 115.35) (width 0.2) (layer "B.Cu") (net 10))
 (segment (start 156 90.25) (end 156 111) (width 0.2) (layer "B.Cu") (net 10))
 (via (at 158.675 91.462) (size 0.6) (drill 0.3) (layers "F.Cu" "B.Cu") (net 11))
 (segment (start 160.2625 114.2625) (end 163.8625 114.2625) (width 0.2) (layer "B.Cu") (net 11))
 (segment (start 158.675 91.462) (end 157.538 91.462) (width 0.2) (layer "B.Cu") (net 11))
 (segment (start 157.538 91.462) (end 156.75 92.25) (width 0.2) (layer "B.Cu") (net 11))
 (segment (start 163.8625 114.2625) (end 164.95 115.35) (width 0.2) (layer "B.Cu") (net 11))
 (segment (start 156.75 92.25) (end 156.75 110.75) (width 0.2) (layer "B.Cu") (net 11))
 (segment (start 156.75 110.75) (end 160.2625 114.2625) (width 0.2) (layer "B.Cu") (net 11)))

